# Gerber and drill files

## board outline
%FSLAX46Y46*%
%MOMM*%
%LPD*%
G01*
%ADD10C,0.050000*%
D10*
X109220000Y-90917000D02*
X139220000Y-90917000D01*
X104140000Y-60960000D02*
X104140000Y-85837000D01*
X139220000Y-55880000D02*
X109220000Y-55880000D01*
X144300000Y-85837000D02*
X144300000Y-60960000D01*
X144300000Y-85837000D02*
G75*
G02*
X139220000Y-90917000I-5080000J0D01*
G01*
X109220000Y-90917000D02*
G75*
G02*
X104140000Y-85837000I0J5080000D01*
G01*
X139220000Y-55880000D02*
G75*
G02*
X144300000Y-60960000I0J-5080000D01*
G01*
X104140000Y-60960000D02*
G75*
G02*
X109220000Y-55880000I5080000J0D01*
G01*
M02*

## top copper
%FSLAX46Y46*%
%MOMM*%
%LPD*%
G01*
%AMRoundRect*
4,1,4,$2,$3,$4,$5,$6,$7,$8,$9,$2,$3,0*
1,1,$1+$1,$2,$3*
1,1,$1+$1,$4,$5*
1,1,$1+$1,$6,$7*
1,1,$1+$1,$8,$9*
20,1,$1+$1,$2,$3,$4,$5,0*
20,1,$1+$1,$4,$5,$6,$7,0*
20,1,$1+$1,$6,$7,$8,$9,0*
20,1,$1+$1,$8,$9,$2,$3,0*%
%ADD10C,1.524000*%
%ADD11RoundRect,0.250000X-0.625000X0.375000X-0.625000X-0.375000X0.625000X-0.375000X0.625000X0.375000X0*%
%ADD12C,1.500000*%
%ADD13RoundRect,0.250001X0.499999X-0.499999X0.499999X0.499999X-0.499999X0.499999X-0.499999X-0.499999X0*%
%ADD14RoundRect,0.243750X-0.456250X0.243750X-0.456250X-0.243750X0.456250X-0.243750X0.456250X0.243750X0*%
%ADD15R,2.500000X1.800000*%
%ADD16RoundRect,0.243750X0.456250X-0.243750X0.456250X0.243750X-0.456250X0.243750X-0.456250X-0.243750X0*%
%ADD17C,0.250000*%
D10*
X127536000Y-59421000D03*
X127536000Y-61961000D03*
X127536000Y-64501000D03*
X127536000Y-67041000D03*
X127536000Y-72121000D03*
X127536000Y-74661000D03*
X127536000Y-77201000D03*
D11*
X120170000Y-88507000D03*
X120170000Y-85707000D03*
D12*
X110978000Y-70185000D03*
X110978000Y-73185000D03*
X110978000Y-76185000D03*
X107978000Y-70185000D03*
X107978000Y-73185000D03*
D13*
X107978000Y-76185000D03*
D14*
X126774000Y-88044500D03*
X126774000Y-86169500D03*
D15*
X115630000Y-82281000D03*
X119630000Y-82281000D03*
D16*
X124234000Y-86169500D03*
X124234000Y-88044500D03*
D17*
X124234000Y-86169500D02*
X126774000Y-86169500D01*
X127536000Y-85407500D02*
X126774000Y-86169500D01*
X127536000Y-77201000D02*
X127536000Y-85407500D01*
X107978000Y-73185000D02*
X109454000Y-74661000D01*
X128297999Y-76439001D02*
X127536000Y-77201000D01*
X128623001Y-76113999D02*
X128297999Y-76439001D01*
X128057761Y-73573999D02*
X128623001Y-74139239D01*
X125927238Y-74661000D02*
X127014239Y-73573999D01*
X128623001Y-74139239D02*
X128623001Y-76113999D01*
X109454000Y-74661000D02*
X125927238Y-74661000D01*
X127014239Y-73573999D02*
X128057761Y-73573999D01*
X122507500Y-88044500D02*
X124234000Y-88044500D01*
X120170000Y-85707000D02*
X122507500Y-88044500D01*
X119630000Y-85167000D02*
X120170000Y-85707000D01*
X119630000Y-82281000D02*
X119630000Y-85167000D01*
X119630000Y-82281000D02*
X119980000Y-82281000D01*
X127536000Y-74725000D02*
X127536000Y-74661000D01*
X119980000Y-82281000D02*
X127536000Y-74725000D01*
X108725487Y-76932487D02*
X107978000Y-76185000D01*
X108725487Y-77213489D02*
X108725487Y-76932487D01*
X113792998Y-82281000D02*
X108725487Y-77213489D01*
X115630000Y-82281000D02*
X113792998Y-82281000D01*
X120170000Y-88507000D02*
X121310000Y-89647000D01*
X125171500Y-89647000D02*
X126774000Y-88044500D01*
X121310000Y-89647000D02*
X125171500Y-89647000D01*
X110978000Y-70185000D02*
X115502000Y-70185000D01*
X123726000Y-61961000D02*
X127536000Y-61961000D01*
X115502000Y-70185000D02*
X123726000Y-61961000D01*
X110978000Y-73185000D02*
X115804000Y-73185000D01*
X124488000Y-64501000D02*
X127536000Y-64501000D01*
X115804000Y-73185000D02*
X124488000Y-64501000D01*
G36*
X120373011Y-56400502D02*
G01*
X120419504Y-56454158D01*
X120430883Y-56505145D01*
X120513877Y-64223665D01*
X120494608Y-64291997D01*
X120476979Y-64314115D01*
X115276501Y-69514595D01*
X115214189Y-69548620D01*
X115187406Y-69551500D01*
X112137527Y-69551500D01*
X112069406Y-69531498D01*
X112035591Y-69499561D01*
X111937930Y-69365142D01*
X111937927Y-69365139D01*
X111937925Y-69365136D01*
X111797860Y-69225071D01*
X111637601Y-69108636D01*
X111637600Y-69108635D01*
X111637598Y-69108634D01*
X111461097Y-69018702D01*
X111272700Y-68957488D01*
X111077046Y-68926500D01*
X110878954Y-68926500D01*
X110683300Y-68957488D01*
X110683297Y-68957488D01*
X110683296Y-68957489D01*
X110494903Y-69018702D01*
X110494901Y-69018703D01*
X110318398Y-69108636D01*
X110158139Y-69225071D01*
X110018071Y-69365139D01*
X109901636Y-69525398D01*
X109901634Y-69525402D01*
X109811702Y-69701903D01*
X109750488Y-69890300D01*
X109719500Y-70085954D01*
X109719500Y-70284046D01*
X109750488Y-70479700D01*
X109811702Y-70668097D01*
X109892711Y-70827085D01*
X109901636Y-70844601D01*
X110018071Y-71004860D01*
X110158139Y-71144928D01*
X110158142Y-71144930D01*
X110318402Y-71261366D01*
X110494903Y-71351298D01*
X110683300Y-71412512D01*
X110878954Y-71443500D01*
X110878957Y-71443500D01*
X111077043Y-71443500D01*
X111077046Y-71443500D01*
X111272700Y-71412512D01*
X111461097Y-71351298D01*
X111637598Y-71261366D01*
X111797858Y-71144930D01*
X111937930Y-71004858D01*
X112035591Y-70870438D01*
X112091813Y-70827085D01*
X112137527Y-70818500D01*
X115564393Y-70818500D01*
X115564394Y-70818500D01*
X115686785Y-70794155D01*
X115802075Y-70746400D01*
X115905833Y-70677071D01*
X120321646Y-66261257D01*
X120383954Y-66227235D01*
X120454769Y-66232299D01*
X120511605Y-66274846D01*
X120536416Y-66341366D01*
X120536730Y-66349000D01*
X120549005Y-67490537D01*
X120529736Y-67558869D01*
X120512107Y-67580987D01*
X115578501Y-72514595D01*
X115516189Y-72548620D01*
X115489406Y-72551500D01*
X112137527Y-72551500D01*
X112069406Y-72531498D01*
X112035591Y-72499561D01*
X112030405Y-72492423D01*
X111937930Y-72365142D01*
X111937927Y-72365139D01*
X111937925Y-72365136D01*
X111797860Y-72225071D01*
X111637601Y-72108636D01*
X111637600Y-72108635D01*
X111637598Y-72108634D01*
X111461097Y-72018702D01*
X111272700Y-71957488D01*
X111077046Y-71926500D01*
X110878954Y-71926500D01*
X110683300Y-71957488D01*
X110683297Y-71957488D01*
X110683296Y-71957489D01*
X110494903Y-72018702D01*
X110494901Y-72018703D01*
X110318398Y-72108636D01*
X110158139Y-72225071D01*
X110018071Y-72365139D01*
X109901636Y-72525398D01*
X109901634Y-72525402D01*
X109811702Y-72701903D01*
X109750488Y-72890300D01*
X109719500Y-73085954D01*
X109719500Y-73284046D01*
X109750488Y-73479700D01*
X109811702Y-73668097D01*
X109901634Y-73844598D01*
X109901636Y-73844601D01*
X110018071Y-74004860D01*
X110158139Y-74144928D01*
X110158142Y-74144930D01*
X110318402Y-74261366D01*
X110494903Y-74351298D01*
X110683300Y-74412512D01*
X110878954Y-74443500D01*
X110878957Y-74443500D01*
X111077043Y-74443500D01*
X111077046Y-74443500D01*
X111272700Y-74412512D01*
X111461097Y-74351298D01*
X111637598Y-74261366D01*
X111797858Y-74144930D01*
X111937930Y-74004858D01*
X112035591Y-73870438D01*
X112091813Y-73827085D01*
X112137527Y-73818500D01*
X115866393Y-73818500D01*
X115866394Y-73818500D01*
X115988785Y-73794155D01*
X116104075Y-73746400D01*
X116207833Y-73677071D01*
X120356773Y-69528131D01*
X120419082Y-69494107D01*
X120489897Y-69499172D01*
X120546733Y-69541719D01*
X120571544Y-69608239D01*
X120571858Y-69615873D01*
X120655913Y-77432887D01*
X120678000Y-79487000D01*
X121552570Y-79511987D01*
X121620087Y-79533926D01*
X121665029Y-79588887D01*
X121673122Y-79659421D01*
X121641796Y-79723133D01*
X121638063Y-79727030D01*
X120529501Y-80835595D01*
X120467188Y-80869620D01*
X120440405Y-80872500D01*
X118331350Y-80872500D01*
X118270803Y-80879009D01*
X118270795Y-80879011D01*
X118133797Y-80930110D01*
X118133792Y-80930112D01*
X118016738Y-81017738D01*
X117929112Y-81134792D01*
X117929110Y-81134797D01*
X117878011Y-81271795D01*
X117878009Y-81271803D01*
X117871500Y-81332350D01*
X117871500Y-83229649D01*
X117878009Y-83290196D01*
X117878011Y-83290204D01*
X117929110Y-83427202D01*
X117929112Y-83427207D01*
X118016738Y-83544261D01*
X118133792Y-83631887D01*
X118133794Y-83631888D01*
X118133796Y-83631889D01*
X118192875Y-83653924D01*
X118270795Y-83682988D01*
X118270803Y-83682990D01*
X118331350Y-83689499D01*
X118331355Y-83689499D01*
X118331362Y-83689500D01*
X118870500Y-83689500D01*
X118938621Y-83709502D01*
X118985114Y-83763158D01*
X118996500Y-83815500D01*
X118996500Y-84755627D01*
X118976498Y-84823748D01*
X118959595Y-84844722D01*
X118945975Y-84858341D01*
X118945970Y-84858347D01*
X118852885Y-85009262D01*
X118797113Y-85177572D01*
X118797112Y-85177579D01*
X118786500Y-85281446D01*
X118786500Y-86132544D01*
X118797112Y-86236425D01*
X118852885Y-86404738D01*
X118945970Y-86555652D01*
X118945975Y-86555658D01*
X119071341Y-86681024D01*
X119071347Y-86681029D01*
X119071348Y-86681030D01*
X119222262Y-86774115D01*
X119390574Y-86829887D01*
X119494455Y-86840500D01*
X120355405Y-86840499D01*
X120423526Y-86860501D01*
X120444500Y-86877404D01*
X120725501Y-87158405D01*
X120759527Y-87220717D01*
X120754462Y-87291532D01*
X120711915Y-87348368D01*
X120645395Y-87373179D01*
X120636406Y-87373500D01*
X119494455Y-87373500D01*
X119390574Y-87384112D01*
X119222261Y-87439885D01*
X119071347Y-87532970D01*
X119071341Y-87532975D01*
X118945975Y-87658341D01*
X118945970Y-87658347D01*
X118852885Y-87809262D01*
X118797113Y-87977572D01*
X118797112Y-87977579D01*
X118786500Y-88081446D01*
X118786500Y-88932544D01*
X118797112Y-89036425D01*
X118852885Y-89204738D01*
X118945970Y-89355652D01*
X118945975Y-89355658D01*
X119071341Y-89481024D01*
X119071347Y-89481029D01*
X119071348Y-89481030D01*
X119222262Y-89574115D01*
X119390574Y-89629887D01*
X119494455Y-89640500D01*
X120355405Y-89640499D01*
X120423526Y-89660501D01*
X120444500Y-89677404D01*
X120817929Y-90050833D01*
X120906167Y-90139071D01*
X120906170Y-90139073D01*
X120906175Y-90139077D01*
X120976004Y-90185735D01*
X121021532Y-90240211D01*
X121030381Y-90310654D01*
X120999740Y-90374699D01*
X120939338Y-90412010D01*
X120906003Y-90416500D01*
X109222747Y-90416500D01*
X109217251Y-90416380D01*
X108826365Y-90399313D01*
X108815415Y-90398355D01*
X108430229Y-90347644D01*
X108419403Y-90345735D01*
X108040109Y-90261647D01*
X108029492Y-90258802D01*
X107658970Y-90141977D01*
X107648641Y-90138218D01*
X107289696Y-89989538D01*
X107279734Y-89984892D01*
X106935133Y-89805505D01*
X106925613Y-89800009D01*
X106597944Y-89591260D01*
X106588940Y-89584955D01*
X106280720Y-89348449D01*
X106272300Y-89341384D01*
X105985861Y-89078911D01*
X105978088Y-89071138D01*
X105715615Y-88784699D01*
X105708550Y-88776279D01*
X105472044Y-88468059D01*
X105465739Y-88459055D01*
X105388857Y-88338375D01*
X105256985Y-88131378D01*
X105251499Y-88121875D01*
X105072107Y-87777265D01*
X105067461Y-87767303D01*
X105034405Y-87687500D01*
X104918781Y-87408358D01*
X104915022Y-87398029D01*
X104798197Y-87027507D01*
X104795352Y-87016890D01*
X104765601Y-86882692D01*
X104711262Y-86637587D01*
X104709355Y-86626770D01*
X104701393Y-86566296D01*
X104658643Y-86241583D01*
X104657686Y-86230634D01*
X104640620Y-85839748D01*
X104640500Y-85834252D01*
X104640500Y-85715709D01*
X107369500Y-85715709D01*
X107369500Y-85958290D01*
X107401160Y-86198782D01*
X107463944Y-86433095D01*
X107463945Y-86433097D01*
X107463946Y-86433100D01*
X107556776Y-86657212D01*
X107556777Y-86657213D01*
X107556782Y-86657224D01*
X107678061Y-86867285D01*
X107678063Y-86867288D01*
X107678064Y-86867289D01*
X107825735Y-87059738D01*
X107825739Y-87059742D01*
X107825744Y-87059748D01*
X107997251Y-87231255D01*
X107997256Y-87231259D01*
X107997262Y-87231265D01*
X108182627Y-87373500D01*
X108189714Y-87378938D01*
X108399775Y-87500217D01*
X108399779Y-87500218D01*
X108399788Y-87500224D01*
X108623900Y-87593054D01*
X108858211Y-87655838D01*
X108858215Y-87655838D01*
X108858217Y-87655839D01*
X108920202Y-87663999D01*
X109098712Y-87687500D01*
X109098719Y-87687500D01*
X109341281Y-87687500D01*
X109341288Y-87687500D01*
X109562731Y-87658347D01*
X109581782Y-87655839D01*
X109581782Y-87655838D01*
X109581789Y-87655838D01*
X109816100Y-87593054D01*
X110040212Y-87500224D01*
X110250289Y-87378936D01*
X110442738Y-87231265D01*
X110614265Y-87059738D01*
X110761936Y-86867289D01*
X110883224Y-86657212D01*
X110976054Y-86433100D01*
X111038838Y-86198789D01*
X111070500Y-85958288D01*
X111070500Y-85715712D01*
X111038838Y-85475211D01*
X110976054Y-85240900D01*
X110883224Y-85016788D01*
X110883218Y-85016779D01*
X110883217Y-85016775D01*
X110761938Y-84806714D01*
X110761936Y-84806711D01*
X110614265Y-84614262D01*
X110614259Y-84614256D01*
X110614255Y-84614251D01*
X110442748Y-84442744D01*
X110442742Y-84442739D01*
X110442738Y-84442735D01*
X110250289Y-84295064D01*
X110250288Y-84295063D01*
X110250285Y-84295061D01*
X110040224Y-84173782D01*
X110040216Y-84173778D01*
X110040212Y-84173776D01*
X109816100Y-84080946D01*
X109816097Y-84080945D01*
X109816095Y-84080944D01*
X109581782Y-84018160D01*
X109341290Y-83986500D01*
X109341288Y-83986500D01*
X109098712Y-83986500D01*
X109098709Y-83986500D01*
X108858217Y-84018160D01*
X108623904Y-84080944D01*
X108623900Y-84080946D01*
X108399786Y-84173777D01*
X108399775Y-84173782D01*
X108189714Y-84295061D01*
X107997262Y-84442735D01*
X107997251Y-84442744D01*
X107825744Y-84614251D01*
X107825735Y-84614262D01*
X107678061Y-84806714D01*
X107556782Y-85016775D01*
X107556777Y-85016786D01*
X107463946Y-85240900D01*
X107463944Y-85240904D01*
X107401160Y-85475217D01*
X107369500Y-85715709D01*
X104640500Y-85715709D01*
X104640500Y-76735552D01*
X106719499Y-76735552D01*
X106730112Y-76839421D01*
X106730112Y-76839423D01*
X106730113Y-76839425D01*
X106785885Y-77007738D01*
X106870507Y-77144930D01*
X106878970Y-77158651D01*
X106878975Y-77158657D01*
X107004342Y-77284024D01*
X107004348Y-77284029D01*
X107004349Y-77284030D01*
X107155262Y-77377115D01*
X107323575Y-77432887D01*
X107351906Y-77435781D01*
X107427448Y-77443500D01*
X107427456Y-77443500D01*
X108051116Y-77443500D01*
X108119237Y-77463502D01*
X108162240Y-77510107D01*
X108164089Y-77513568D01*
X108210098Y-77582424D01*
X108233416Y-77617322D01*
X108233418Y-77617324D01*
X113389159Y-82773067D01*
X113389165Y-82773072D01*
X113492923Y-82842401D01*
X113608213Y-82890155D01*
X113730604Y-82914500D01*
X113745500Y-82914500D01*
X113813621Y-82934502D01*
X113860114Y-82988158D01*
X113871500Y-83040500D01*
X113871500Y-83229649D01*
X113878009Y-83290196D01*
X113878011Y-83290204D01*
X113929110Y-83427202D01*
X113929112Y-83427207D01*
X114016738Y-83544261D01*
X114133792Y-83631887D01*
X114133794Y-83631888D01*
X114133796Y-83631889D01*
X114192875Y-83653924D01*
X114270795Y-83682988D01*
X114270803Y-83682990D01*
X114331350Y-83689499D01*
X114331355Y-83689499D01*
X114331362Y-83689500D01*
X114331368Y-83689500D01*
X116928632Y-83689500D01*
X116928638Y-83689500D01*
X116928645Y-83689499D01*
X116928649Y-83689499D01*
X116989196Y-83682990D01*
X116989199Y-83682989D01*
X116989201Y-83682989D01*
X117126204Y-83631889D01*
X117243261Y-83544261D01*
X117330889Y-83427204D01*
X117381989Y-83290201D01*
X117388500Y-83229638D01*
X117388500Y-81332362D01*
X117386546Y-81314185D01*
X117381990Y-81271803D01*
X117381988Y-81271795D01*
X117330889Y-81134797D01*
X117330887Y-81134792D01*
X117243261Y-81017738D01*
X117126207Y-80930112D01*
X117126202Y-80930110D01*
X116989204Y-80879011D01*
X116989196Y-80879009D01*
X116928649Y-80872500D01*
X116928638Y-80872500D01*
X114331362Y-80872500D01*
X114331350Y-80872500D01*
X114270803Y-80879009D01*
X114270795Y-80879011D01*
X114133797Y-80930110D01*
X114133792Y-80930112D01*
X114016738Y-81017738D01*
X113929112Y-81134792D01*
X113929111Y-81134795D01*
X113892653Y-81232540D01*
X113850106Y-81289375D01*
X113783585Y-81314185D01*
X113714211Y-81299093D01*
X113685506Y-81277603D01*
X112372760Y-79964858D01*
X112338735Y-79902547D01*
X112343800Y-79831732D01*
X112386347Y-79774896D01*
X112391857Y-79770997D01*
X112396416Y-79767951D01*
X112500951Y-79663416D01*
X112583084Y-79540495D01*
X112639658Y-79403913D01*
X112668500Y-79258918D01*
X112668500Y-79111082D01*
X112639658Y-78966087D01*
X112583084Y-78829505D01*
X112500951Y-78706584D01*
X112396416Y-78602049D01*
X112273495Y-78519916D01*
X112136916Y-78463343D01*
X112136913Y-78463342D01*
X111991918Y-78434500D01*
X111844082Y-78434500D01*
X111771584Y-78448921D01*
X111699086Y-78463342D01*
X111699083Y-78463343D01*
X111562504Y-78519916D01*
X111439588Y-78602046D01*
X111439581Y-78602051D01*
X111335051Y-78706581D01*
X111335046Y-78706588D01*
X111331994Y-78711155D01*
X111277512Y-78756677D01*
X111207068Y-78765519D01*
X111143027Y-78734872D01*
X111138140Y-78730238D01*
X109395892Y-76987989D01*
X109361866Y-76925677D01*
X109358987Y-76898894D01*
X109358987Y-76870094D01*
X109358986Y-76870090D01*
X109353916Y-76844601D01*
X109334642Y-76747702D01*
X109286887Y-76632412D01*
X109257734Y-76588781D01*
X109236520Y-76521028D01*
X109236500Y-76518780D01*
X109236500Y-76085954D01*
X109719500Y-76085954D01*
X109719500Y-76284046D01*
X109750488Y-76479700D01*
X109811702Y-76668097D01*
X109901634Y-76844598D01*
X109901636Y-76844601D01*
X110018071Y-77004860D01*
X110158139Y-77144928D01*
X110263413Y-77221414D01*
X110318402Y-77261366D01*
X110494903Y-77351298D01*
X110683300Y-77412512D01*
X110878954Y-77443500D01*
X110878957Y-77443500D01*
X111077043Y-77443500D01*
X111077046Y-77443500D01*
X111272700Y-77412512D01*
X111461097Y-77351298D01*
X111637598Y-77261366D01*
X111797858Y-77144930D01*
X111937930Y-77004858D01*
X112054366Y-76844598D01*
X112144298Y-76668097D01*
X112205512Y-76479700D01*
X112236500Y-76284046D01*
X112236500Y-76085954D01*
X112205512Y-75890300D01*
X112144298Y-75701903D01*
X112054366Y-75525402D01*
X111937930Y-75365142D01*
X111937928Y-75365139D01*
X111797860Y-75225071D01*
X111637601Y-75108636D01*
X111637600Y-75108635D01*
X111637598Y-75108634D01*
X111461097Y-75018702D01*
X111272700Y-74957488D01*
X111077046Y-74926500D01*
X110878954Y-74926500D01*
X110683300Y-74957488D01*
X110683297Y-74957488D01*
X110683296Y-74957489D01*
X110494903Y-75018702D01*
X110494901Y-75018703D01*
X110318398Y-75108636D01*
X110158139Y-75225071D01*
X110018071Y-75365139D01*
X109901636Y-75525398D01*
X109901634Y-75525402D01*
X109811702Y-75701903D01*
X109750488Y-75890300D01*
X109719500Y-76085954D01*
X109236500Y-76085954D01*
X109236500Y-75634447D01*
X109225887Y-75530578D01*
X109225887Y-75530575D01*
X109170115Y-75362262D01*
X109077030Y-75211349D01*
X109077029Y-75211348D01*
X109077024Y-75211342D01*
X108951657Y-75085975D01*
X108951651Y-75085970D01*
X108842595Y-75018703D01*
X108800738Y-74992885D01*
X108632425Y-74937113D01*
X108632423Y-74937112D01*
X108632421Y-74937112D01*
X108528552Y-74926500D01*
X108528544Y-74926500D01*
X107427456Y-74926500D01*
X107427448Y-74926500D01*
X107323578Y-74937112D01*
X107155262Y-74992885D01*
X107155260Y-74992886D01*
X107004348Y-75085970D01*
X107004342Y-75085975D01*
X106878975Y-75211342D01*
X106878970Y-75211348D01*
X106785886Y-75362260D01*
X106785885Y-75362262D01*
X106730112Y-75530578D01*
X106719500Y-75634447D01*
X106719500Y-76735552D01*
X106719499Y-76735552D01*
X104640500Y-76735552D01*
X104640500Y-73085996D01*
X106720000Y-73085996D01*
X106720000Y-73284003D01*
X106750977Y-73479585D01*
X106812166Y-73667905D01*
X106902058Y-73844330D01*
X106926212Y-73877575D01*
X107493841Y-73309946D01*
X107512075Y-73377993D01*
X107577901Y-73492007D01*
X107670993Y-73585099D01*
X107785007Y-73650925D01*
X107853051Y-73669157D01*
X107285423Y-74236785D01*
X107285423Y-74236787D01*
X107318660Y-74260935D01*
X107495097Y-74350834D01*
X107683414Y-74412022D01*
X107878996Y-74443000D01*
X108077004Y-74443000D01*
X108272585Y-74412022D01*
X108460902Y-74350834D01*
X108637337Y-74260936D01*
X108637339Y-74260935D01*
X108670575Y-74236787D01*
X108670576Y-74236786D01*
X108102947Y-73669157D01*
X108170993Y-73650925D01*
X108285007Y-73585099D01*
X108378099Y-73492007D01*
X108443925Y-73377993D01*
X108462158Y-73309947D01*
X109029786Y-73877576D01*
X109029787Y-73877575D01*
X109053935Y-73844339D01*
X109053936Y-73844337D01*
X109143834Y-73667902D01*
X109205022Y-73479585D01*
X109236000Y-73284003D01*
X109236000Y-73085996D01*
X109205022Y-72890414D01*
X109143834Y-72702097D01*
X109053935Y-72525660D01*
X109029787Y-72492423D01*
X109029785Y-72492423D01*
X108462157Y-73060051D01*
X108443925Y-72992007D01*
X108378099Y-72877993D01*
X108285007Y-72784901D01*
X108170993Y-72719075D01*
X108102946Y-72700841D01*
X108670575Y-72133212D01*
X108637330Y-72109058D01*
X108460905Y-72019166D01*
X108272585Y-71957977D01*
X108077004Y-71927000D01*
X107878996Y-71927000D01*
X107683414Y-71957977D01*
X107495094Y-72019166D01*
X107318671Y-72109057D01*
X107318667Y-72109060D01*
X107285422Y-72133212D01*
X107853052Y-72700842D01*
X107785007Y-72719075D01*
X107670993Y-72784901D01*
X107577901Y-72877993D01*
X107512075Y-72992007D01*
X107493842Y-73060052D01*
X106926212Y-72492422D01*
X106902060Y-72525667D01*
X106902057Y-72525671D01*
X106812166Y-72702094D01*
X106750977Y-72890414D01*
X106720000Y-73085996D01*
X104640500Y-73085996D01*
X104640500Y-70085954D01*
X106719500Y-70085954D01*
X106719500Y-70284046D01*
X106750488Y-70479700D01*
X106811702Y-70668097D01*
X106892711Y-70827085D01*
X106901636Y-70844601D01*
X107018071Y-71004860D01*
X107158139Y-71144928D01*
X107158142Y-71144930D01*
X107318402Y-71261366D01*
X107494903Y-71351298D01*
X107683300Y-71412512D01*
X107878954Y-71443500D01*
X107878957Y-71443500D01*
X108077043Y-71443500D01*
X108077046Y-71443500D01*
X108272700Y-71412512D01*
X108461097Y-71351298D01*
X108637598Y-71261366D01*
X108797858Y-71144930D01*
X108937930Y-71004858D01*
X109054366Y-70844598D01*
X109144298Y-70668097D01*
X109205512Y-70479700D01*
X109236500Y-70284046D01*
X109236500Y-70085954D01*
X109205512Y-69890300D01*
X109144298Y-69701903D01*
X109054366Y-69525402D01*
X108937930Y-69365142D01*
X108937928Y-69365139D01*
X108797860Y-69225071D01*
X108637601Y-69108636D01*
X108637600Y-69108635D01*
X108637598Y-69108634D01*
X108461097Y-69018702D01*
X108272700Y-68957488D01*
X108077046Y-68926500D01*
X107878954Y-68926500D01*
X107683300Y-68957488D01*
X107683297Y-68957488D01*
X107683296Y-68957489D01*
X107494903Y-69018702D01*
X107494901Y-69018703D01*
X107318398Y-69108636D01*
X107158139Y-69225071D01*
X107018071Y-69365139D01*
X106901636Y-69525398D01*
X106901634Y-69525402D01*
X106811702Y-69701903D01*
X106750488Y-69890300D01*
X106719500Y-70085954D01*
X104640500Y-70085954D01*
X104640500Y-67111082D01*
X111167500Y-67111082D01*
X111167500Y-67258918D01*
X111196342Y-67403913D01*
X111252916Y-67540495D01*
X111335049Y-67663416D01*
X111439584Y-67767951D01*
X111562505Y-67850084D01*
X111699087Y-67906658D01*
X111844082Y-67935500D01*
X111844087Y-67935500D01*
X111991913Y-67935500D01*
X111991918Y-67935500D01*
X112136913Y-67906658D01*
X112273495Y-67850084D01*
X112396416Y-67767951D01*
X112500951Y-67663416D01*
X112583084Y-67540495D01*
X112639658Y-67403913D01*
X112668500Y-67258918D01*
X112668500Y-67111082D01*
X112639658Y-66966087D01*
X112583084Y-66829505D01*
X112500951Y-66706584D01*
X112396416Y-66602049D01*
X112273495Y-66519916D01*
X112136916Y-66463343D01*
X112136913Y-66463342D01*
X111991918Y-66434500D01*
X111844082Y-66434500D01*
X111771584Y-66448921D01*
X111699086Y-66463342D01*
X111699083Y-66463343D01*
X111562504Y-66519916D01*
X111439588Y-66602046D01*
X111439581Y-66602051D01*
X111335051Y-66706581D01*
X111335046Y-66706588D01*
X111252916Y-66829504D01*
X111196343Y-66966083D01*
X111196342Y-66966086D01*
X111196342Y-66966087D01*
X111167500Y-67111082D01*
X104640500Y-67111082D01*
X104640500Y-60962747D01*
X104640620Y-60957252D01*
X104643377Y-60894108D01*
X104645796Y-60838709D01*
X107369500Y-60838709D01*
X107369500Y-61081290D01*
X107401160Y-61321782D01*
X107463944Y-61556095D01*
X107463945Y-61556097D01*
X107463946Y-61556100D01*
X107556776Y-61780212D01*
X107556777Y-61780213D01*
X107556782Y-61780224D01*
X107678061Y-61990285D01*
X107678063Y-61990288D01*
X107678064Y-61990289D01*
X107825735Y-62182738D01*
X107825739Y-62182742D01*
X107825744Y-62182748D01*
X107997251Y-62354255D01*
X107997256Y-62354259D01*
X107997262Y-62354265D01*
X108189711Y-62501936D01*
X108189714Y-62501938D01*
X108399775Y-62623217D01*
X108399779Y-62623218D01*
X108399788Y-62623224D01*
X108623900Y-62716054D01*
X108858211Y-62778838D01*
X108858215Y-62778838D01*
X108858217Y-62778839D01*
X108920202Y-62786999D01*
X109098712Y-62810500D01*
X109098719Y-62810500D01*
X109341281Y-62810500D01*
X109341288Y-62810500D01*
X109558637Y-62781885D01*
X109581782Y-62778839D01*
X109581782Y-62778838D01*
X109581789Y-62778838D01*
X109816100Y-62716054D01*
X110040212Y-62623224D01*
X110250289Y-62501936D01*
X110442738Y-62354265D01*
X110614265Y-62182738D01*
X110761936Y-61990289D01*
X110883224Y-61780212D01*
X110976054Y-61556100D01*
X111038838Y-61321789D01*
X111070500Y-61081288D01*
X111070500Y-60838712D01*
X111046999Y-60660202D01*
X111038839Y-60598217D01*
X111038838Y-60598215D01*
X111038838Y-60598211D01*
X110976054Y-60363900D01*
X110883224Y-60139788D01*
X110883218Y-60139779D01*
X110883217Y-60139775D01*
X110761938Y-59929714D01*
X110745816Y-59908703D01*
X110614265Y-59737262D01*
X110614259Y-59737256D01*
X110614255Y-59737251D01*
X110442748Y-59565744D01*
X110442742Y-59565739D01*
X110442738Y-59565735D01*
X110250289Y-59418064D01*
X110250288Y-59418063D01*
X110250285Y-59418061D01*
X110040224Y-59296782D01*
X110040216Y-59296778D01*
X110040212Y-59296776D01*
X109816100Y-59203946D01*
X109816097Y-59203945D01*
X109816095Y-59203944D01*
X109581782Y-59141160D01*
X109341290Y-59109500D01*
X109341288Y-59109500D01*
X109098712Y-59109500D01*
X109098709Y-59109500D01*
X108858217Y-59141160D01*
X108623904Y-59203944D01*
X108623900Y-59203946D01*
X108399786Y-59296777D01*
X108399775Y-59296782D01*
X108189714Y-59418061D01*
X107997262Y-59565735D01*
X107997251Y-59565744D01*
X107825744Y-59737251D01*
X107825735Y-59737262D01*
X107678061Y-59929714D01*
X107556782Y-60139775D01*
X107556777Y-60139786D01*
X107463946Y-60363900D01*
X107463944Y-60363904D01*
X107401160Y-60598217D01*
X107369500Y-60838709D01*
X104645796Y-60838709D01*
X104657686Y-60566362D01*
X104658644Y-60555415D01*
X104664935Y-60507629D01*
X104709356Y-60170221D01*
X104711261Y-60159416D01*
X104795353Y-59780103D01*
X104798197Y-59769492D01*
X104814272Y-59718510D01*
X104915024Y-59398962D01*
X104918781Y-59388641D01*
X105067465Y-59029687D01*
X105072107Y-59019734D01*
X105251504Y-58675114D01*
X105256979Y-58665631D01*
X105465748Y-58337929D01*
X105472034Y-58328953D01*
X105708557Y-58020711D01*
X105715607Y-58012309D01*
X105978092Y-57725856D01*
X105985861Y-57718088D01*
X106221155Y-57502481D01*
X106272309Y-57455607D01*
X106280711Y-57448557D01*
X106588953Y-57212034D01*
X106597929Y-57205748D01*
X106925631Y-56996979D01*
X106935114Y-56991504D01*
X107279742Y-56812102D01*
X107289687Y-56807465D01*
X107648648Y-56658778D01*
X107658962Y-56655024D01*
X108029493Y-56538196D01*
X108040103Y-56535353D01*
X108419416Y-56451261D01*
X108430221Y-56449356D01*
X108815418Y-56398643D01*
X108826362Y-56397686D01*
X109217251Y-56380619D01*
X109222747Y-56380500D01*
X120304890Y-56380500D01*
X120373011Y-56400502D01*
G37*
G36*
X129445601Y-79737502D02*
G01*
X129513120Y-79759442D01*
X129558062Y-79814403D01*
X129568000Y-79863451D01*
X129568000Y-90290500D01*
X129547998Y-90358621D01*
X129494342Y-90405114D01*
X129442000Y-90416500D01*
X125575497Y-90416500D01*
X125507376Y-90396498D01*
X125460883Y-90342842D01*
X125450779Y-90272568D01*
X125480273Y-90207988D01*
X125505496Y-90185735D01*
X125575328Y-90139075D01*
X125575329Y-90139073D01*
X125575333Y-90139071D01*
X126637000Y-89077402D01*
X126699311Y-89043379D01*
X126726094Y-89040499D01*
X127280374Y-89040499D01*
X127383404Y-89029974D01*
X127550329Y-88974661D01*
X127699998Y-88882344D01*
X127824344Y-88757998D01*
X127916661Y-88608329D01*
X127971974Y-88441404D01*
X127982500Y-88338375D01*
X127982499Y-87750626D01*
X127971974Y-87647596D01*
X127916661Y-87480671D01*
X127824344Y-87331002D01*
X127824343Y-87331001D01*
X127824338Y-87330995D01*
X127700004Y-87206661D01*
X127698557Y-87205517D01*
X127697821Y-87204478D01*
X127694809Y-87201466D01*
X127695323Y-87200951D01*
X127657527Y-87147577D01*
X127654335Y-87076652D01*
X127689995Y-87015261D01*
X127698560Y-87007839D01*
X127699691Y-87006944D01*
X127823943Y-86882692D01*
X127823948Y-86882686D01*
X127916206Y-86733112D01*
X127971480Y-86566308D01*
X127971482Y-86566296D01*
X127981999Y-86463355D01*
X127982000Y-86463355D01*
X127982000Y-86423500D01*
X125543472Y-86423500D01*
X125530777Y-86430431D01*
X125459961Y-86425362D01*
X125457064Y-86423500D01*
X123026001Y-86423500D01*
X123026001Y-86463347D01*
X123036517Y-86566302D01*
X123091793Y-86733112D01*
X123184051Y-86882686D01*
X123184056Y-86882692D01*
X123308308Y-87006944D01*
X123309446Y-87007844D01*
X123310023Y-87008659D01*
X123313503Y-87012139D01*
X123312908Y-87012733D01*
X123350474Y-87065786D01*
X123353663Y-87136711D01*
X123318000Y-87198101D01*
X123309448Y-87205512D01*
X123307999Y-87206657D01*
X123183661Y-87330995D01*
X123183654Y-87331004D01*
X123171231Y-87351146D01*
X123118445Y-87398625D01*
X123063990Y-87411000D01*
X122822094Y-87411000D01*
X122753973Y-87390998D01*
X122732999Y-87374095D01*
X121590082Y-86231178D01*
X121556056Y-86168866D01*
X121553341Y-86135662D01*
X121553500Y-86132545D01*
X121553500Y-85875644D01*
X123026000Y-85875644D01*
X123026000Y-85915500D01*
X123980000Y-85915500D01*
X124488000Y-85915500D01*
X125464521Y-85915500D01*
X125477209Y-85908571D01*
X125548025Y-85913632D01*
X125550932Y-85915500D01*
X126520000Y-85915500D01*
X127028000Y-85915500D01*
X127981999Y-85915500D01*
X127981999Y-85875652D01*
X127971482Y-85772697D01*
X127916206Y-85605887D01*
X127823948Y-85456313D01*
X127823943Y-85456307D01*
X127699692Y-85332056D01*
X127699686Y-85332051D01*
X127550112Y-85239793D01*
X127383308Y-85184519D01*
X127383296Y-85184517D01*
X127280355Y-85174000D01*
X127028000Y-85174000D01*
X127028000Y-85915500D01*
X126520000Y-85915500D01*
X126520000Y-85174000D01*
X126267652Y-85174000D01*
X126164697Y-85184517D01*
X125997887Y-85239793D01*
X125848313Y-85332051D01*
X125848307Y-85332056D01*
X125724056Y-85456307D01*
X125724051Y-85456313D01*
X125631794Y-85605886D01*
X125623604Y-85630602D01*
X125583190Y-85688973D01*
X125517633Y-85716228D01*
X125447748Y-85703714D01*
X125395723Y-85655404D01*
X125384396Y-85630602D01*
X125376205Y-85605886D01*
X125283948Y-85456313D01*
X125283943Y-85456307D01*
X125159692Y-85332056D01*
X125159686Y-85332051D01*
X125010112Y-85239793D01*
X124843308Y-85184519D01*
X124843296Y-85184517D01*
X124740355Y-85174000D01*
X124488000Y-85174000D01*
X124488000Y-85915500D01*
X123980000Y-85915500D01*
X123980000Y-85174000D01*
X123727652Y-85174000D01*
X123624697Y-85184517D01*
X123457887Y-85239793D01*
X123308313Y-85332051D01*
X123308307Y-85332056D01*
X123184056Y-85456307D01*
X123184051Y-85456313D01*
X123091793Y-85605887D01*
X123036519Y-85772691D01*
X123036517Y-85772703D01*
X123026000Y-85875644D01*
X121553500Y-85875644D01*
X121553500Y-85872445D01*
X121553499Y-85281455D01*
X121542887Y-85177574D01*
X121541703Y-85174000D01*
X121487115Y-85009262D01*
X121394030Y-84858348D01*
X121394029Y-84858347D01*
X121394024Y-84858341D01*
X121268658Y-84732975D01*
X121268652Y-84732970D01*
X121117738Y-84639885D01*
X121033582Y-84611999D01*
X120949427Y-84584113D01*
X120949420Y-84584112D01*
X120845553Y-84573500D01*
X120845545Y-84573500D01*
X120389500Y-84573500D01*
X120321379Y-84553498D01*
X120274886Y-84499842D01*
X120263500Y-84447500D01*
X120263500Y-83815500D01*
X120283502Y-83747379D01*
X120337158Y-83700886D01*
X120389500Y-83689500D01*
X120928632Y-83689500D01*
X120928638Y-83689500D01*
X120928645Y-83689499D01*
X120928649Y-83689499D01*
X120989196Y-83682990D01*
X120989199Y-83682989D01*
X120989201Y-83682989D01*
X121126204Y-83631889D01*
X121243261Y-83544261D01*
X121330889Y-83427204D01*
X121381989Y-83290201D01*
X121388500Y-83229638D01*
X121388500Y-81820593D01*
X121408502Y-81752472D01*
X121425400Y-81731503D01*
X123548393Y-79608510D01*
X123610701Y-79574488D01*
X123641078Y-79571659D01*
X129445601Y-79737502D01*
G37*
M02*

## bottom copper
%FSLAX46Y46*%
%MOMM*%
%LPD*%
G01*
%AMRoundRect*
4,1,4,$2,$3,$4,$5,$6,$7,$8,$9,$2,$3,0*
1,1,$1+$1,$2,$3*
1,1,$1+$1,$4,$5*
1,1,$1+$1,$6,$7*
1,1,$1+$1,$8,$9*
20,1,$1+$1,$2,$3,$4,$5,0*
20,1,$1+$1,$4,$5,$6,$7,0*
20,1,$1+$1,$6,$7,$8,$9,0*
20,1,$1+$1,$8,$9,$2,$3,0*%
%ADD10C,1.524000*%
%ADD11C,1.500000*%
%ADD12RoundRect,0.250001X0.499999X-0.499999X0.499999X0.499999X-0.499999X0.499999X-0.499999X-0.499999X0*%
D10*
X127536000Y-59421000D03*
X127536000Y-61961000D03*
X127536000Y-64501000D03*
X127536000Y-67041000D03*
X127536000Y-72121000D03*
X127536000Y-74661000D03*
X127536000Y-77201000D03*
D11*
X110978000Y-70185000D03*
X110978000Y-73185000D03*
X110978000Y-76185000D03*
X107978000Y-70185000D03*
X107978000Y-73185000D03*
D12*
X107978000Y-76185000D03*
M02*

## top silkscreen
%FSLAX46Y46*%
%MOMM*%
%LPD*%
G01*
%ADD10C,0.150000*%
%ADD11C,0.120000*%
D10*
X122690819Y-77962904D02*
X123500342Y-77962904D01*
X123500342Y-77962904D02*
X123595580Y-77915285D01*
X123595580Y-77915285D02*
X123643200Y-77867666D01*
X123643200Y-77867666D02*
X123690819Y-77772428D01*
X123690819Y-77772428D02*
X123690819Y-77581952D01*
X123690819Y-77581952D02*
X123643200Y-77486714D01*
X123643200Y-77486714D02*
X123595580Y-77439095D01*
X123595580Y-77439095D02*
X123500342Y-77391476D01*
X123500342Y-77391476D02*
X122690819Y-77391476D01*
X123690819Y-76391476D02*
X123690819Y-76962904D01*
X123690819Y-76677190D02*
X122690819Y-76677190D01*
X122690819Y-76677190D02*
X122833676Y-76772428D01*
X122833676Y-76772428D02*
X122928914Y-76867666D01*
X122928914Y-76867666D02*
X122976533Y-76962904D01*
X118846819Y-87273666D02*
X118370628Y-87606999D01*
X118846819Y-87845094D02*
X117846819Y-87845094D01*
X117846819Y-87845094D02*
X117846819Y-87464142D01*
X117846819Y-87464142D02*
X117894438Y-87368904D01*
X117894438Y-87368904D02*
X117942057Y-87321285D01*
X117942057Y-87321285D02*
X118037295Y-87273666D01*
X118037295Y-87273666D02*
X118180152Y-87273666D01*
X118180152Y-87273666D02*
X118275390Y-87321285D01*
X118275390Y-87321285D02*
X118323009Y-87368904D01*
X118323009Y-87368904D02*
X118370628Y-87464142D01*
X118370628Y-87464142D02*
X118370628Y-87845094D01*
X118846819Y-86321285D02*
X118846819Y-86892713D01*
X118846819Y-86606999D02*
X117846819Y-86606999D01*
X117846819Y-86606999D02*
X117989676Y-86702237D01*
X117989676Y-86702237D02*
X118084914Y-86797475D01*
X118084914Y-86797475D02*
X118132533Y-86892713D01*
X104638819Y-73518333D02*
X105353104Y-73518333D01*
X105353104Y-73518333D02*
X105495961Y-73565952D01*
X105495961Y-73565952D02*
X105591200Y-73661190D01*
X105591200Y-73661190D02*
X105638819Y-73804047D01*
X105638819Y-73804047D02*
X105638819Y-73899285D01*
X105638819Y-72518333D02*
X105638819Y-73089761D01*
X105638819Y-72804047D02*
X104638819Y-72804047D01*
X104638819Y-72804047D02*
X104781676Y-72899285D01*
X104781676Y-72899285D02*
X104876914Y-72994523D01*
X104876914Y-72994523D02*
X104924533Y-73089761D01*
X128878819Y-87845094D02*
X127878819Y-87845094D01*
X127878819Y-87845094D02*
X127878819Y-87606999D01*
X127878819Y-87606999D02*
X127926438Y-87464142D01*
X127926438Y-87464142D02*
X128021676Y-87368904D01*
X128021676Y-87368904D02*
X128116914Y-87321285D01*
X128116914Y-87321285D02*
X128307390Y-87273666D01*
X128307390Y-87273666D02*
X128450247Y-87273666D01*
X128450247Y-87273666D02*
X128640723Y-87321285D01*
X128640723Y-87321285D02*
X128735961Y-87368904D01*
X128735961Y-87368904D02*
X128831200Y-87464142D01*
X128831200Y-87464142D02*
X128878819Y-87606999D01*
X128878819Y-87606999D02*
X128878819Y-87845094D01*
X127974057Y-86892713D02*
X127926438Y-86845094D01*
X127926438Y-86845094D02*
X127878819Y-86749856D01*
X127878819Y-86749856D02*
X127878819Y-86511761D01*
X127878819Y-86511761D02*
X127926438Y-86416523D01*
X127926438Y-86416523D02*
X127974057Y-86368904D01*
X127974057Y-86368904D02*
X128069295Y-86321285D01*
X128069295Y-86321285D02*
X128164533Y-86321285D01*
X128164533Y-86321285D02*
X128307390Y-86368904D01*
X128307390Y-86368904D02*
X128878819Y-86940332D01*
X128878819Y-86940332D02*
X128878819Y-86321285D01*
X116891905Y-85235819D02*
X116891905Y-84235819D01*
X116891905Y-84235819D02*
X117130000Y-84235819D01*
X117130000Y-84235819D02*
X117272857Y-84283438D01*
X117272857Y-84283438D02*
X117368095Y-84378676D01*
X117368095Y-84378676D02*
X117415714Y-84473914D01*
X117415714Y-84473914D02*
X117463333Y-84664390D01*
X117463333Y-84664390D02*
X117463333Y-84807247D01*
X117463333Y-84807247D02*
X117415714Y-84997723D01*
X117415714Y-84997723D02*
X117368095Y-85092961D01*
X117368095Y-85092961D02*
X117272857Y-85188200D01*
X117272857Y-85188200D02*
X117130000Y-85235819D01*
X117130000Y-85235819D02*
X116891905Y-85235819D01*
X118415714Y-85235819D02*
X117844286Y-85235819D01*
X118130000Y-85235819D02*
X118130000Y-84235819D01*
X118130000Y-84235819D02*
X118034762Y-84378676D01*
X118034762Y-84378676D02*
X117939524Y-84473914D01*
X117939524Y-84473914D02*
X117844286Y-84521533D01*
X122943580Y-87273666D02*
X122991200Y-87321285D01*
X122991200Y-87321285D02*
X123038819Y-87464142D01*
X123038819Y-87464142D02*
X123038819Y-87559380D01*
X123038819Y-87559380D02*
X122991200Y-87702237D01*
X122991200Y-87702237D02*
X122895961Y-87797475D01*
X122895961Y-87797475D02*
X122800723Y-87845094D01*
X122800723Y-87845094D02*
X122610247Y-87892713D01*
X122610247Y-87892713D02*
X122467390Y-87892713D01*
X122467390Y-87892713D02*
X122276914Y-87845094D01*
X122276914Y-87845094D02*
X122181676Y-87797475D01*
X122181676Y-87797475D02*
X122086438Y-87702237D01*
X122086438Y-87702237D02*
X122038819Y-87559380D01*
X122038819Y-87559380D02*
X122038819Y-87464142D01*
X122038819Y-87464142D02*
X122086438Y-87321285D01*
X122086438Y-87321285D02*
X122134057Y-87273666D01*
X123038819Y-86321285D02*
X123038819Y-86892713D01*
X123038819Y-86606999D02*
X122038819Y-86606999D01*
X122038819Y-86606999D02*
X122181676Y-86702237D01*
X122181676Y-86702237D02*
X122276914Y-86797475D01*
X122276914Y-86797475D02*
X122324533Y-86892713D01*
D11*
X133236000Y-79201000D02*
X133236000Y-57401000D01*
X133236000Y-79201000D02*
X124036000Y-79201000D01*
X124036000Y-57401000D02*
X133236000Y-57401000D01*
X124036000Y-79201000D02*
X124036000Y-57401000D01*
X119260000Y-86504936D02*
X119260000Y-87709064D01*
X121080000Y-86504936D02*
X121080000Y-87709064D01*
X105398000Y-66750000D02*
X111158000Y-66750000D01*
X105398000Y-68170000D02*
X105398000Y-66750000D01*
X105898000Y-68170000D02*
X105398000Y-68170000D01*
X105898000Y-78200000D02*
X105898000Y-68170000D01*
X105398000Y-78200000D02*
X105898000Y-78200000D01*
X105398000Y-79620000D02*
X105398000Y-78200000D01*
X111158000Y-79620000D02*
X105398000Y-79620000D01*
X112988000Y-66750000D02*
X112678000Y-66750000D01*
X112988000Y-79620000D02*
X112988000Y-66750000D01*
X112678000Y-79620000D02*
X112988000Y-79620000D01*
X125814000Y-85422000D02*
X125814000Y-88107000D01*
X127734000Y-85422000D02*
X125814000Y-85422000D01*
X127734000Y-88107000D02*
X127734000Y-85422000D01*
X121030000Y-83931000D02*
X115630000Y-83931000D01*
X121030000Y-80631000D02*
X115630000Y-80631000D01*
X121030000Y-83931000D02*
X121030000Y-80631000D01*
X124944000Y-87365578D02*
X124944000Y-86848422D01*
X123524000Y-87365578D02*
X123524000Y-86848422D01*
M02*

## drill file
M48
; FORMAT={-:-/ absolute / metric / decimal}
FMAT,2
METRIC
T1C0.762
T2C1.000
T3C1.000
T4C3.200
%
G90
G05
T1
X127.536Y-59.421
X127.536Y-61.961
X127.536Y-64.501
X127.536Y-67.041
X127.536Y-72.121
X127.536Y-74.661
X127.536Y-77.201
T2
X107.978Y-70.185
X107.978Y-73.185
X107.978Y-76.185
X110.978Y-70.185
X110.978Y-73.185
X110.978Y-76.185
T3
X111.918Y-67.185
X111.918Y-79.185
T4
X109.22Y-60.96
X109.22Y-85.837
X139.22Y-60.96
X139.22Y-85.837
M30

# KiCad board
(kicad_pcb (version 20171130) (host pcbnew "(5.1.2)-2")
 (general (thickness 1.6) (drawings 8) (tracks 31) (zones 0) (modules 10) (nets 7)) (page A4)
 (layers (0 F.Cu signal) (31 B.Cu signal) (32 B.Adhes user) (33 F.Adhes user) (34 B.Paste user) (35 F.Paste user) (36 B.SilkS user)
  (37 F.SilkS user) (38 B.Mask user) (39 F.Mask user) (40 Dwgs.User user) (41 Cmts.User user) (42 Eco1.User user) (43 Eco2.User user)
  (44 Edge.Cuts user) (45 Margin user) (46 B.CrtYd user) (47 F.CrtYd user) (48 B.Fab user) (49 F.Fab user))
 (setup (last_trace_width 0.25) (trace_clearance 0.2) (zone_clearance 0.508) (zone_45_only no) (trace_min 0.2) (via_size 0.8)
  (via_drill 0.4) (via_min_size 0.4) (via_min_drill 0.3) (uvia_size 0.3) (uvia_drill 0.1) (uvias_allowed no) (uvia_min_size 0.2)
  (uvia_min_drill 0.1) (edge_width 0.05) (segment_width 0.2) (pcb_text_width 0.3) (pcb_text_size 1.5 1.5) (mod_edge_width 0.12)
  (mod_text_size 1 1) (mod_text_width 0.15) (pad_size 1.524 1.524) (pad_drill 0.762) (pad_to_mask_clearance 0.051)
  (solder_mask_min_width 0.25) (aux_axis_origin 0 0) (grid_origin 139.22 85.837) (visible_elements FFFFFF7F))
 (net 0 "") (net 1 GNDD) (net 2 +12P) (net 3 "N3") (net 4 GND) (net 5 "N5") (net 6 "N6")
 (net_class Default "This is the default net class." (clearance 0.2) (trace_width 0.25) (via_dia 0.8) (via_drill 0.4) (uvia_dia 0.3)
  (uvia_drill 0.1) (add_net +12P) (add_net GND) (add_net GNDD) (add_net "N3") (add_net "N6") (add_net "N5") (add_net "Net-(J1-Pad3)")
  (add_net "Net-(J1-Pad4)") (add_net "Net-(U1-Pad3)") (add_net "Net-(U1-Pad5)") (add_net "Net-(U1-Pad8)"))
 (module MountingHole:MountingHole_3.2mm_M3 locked (layer F.Cu) (at 139.22 85.837)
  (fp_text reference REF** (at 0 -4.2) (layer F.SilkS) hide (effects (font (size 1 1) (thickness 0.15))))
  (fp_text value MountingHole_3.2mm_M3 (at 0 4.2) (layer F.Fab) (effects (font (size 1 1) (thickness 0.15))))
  (pad 1 np_thru_hole circle (at 0 0) (size 3.2 3.2) (drill 3.2) (layers *.Cu *.Mask)))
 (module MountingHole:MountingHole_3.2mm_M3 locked (layer F.Cu) (at 109.22 85.837)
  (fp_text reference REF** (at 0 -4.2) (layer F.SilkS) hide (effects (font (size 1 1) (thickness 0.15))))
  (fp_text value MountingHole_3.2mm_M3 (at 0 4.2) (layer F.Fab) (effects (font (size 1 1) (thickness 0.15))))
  (pad 1 np_thru_hole circle (at 0 0) (size 3.2 3.2) (drill 3.2) (layers *.Cu *.Mask)))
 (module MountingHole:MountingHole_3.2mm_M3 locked (layer F.Cu) (at 109.22 60.96)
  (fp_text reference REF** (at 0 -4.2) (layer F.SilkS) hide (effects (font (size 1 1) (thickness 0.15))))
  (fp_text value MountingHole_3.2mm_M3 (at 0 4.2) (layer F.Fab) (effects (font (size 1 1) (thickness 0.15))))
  (pad 1 np_thru_hole circle (at 0 0) (size 3.2 3.2) (drill 3.2) (layers *.Cu *.Mask)))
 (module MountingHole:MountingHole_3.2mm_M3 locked (layer F.Cu) (at 139.22 60.96)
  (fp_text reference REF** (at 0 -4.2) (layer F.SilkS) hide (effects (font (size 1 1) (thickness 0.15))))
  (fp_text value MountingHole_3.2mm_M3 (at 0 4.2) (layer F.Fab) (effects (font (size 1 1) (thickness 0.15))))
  (pad 1 np_thru_hole circle (at 0 0) (size 3.2 3.2) (drill 3.2) (layers *.Cu *.Mask)))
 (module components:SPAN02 (layer F.Cu) (at 127.536 77.201 90)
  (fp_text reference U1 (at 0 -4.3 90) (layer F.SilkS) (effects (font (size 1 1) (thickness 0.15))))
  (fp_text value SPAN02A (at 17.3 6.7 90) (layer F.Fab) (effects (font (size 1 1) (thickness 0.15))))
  (fp_line (start -2 5.7) (end 19.8 5.7) (layer F.SilkS) (width 0.12))
  (fp_line (start -2 5.7) (end -2 -3.5) (layer F.SilkS) (width 0.12))
  (fp_line (start 19.8 -3.5) (end 19.8 5.7) (layer F.SilkS) (width 0.12))
  (fp_line (start -2 -3.5) (end 19.8 -3.5) (layer F.SilkS) (width 0.12))
  (pad 8 thru_hole circle (at 17.78 0 90) (size 1.524 1.524) (drill 0.762) (layers *.Cu *.Mask))
  (pad 7 thru_hole circle (at 15.24 0 90) (size 1.524 1.524) (drill 0.762) (layers *.Cu *.Mask) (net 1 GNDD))
  (pad 6 thru_hole circle (at 12.7 0 90) (size 1.524 1.524) (drill 0.762) (layers *.Cu *.Mask) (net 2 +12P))
  (pad 5 thru_hole circle (at 10.16 0 90) (size 1.524 1.524) (drill 0.762) (layers *.Cu *.Mask))
  (pad 3 thru_hole circle (at 5.08 0 90) (size 1.524 1.524) (drill 0.762) (layers *.Cu *.Mask))
  (pad 2 thru_hole circle (at 2.54 0 90) (size 1.524 1.524) (drill 0.762) (layers *.Cu *.Mask) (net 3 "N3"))
  (pad 1 thru_hole circle (at 0 0 90) (size 1.524 1.524) (drill 0.762) (layers *.Cu *.Mask) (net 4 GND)))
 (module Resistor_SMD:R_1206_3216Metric (layer F.Cu) (at 120.17 87.107 270)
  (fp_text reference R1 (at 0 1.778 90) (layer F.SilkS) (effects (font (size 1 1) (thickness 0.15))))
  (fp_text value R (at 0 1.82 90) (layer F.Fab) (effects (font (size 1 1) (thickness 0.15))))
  (fp_line (start -0.602064 0.91) (end 0.602064 0.91) (layer F.SilkS) (width 0.12))
  (fp_line (start -0.602064 -0.91) (end 0.602064 -0.91) (layer F.SilkS) (width 0.12))
  (pad 2 smd roundrect (at 1.4 0 270) (size 1.25 1.75) (layers F.Cu F.Paste F.Mask) (roundrect_rratio 0.2) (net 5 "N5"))
  (pad 1 smd roundrect (at -1.4 0 270) (size 1.25 1.75) (layers F.Cu F.Paste F.Mask) (roundrect_rratio 0.2) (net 3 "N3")))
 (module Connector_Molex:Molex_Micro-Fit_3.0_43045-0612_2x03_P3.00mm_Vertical (layer F.Cu) (at 107.978 76.185 90)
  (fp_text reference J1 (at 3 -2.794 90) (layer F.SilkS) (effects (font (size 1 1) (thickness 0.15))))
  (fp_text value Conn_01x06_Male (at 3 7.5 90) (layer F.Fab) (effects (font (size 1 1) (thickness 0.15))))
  (fp_line (start 9.435 -2.58) (end 9.435 3.18) (layer F.SilkS) (width 0.12))
  (fp_line (start 8.015 -2.58) (end 9.435 -2.58) (layer F.SilkS) (width 0.12))
  (fp_line (start 8.015 -2.08) (end 8.015 -2.58) (layer F.SilkS) (width 0.12))
  (fp_line (start -2.015 -2.08) (end 8.015 -2.08) (layer F.SilkS) (width 0.12))
  (fp_line (start -2.015 -2.58) (end -2.015 -2.08) (layer F.SilkS) (width 0.12))
  (fp_line (start -3.435 -2.58) (end -2.015 -2.58) (layer F.SilkS) (width 0.12))
  (fp_line (start -3.435 3.18) (end -3.435 -2.58) (layer F.SilkS) (width 0.12))
  (fp_line (start 9.435 5.01) (end 9.435 4.7) (layer F.SilkS) (width 0.12))
  (fp_line (start -3.435 5.01) (end 9.435 5.01) (layer F.SilkS) (width 0.12))
  (fp_line (start -3.435 4.7) (end -3.435 5.01) (layer F.SilkS) (width 0.12))
  (pad 6 thru_hole circle (at 6 3 90) (size 1.5 1.5) (drill 1) (layers *.Cu *.Mask) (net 1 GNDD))
  (pad 5 thru_hole circle (at 3 3 90) (size 1.5 1.5) (drill 1) (layers *.Cu *.Mask) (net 2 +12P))
  (pad 4 thru_hole circle (at 0 3 90) (size 1.5 1.5) (drill 1) (layers *.Cu *.Mask))
  (pad 3 thru_hole circle (at 6 0 90) (size 1.5 1.5) (drill 1) (layers *.Cu *.Mask))
  (pad 2 thru_hole circle (at 3 0 90) (size 1.5 1.5) (drill 1) (layers *.Cu *.Mask) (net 4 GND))
  (pad 1 thru_hole roundrect (at 0 0 90) (size 1.5 1.5) (drill 1) (layers *.Cu *.Mask) (roundrect_rratio 0.166667) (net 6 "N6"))
  (pad "" np_thru_hole circle (at 9 3.94 90) (size 1 1) (drill 1) (layers *.Cu *.Mask))
  (pad "" np_thru_hole circle (at -3 3.94 90) (size 1 1) (drill 1) (layers *.Cu *.Mask)))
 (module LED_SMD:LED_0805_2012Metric (layer F.Cu) (at 126.774 87.107 270)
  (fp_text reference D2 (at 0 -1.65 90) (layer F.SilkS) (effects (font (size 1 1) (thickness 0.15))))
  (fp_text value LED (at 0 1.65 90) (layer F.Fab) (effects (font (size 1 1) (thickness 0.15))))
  (fp_line (start -1.685 0.96) (end 1 0.96) (layer F.SilkS) (width 0.12))
  (fp_line (start -1.685 -0.96) (end -1.685 0.96) (layer F.SilkS) (width 0.12))
  (fp_line (start 1 -0.96) (end -1.685 -0.96) (layer F.SilkS) (width 0.12))
  (pad 2 smd roundrect (at 0.9375 0 270) (size 0.975 1.4) (layers F.Cu F.Paste F.Mask) (roundrect_rratio 0.25) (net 5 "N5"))
  (pad 1 smd roundrect (at -0.9375 0 270) (size 0.975 1.4) (layers F.Cu F.Paste F.Mask) (roundrect_rratio 0.25) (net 4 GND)))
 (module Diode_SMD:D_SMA (layer F.Cu) (at 117.63 82.281 180)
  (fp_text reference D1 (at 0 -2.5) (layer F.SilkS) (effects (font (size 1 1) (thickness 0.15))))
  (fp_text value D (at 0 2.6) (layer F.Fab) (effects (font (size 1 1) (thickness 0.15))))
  (fp_line (start -3.4 -1.65) (end 2 -1.65) (layer F.SilkS) (width 0.12))
  (fp_line (start -3.4 1.65) (end 2 1.65) (layer F.SilkS) (width 0.12))
  (fp_line (start -3.4 -1.65) (end -3.4 1.65) (layer F.SilkS) (width 0.12))
  (pad 2 smd rect (at 2 0 180) (size 2.5 1.8) (layers F.Cu F.Paste F.Mask) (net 6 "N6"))
  (pad 1 smd rect (at -2 0 180) (size 2.5 1.8) (layers F.Cu F.Paste F.Mask) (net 3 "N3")))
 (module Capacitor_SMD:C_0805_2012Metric (layer F.Cu) (at 124.234 87.107 90)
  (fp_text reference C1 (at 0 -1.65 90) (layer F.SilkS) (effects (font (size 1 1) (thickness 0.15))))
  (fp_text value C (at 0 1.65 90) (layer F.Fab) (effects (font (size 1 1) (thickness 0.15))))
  (fp_line (start -0.258578 0.71) (end 0.258578 0.71) (layer F.SilkS) (width 0.12))
  (fp_line (start -0.258578 -0.71) (end 0.258578 -0.71) (layer F.SilkS) (width 0.12))
  (pad 2 smd roundrect (at 0.9375 0 90) (size 0.975 1.4) (layers F.Cu F.Paste F.Mask) (roundrect_rratio 0.25) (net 4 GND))
  (pad 1 smd roundrect (at -0.9375 0 90) (size 0.975 1.4) (layers F.Cu F.Paste F.Mask) (roundrect_rratio 0.25) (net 3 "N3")))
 (gr_line (start 109.22 90.917) (end 139.22 90.917) (layer Edge.Cuts) (width 0.05))
 (gr_line (start 104.14 60.96) (end 104.14 85.837) (layer Edge.Cuts) (width 0.05))
 (gr_line (start 139.22 55.88) (end 109.22 55.88) (layer Edge.Cuts) (width 0.05))
 (gr_line (start 144.3 85.837) (end 144.3 60.96) (layer Edge.Cuts) (width 0.05))
 (gr_arc (start 139.22 85.837) (end 139.22 90.917) (angle -90) (layer Edge.Cuts) (width 0.05))
 (gr_arc (start 109.22 85.837) (end 104.14 85.837) (angle -90) (layer Edge.Cuts) (width 0.05))
 (gr_arc (start 139.22 60.96) (end 144.3 60.96) (angle -90) (layer Edge.Cuts) (width 0.05))
 (gr_arc (start 109.22 60.96) (end 109.22 55.88) (angle -90) (layer Edge.Cuts) (width 0.05))
 (segment (start 124.234 86.1695) (end 126.774 86.1695) (width 0.25) (layer F.Cu) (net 4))
 (segment (start 127.536 85.4075) (end 126.774 86.1695) (width 0.25) (layer F.Cu) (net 4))
 (segment (start 127.536 77.201) (end 127.536 85.4075) (width 0.25) (layer F.Cu) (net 4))
 (segment (start 107.978 73.185) (end 109.454 74.661) (width 0.25) (layer F.Cu) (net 4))
 (segment (start 128.297999 76.439001) (end 127.536 77.201) (width 0.25) (layer F.Cu) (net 4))
 (segment (start 128.623001 76.113999) (end 128.297999 76.439001) (width 0.25) (layer F.Cu) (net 4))
 (segment (start 128.057761 73.573999) (end 128.623001 74.139239) (width 0.25) (layer F.Cu) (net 4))
 (segment (start 125.927238 74.661) (end 127.014239 73.573999) (width 0.25) (layer F.Cu) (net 4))
 (segment (start 128.623001 74.139239) (end 128.623001 76.113999) (width 0.25) (layer F.Cu) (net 4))
 (segment (start 109.454 74.661) (end 125.927238 74.661) (width 0.25) (layer F.Cu) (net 4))
 (segment (start 127.014239 73.573999) (end 128.057761 73.573999) (width 0.25) (layer F.Cu) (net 4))
 (segment (start 122.5075 88.0445) (end 124.234 88.0445) (width 0.25) (layer F.Cu) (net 3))
 (segment (start 120.17 85.707) (end 122.5075 88.0445) (width 0.25) (layer F.Cu) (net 3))
 (segment (start 119.63 85.167) (end 120.17 85.707) (width 0.25) (layer F.Cu) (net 3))
 (segment (start 119.63 82.281) (end 119.63 85.167) (width 0.25) (layer F.Cu) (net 3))
 (segment (start 119.63 82.281) (end 119.98 82.281) (width 0.25) (layer F.Cu) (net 3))
 (segment (start 127.536 74.725) (end 127.536 74.661) (width 0.25) (layer F.Cu) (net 3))
 (segment (start 119.98 82.281) (end 127.536 74.725) (width 0.25) (layer F.Cu) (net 3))
 (segment (start 108.725487 76.932487) (end 107.978 76.185) (width 0.25) (layer F.Cu) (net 6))
 (segment (start 108.725487 77.213489) (end 108.725487 76.932487) (width 0.25) (layer F.Cu) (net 6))
 (segment (start 113.792998 82.281) (end 108.725487 77.213489) (width 0.25) (layer F.Cu) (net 6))
 (segment (start 115.63 82.281) (end 113.792998 82.281) (width 0.25) (layer F.Cu) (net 6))
 (segment (start 120.17 88.507) (end 121.31 89.647) (width 0.25) (layer F.Cu) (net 5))
 (segment (start 125.1715 89.647) (end 126.774 88.0445) (width 0.25) (layer F.Cu) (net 5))
 (segment (start 121.31 89.647) (end 125.1715 89.647) (width 0.25) (layer F.Cu) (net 5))
 (segment (start 110.978 70.185) (end 115.502 70.185) (width 0.25) (layer F.Cu) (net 1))
 (segment (start 123.726 61.961) (end 127.536 61.961) (width 0.25) (layer F.Cu) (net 1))
 (segment (start 115.502 70.185) (end 123.726 61.961) (width 0.25) (layer F.Cu) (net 1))
 (segment (start 110.978 73.185) (end 115.804 73.185) (width 0.25) (layer F.Cu) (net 2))
 (segment (start 124.488 64.501) (end 127.536 64.501) (width 0.25) (layer F.Cu) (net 2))
 (segment (start 115.804 73.185) (end 124.488 64.501) (width 0.25) (layer F.Cu) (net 2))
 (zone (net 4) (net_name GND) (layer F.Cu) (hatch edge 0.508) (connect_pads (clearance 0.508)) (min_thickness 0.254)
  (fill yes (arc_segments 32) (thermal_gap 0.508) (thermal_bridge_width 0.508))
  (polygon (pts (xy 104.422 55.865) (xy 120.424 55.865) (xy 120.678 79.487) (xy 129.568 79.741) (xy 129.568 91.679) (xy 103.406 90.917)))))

